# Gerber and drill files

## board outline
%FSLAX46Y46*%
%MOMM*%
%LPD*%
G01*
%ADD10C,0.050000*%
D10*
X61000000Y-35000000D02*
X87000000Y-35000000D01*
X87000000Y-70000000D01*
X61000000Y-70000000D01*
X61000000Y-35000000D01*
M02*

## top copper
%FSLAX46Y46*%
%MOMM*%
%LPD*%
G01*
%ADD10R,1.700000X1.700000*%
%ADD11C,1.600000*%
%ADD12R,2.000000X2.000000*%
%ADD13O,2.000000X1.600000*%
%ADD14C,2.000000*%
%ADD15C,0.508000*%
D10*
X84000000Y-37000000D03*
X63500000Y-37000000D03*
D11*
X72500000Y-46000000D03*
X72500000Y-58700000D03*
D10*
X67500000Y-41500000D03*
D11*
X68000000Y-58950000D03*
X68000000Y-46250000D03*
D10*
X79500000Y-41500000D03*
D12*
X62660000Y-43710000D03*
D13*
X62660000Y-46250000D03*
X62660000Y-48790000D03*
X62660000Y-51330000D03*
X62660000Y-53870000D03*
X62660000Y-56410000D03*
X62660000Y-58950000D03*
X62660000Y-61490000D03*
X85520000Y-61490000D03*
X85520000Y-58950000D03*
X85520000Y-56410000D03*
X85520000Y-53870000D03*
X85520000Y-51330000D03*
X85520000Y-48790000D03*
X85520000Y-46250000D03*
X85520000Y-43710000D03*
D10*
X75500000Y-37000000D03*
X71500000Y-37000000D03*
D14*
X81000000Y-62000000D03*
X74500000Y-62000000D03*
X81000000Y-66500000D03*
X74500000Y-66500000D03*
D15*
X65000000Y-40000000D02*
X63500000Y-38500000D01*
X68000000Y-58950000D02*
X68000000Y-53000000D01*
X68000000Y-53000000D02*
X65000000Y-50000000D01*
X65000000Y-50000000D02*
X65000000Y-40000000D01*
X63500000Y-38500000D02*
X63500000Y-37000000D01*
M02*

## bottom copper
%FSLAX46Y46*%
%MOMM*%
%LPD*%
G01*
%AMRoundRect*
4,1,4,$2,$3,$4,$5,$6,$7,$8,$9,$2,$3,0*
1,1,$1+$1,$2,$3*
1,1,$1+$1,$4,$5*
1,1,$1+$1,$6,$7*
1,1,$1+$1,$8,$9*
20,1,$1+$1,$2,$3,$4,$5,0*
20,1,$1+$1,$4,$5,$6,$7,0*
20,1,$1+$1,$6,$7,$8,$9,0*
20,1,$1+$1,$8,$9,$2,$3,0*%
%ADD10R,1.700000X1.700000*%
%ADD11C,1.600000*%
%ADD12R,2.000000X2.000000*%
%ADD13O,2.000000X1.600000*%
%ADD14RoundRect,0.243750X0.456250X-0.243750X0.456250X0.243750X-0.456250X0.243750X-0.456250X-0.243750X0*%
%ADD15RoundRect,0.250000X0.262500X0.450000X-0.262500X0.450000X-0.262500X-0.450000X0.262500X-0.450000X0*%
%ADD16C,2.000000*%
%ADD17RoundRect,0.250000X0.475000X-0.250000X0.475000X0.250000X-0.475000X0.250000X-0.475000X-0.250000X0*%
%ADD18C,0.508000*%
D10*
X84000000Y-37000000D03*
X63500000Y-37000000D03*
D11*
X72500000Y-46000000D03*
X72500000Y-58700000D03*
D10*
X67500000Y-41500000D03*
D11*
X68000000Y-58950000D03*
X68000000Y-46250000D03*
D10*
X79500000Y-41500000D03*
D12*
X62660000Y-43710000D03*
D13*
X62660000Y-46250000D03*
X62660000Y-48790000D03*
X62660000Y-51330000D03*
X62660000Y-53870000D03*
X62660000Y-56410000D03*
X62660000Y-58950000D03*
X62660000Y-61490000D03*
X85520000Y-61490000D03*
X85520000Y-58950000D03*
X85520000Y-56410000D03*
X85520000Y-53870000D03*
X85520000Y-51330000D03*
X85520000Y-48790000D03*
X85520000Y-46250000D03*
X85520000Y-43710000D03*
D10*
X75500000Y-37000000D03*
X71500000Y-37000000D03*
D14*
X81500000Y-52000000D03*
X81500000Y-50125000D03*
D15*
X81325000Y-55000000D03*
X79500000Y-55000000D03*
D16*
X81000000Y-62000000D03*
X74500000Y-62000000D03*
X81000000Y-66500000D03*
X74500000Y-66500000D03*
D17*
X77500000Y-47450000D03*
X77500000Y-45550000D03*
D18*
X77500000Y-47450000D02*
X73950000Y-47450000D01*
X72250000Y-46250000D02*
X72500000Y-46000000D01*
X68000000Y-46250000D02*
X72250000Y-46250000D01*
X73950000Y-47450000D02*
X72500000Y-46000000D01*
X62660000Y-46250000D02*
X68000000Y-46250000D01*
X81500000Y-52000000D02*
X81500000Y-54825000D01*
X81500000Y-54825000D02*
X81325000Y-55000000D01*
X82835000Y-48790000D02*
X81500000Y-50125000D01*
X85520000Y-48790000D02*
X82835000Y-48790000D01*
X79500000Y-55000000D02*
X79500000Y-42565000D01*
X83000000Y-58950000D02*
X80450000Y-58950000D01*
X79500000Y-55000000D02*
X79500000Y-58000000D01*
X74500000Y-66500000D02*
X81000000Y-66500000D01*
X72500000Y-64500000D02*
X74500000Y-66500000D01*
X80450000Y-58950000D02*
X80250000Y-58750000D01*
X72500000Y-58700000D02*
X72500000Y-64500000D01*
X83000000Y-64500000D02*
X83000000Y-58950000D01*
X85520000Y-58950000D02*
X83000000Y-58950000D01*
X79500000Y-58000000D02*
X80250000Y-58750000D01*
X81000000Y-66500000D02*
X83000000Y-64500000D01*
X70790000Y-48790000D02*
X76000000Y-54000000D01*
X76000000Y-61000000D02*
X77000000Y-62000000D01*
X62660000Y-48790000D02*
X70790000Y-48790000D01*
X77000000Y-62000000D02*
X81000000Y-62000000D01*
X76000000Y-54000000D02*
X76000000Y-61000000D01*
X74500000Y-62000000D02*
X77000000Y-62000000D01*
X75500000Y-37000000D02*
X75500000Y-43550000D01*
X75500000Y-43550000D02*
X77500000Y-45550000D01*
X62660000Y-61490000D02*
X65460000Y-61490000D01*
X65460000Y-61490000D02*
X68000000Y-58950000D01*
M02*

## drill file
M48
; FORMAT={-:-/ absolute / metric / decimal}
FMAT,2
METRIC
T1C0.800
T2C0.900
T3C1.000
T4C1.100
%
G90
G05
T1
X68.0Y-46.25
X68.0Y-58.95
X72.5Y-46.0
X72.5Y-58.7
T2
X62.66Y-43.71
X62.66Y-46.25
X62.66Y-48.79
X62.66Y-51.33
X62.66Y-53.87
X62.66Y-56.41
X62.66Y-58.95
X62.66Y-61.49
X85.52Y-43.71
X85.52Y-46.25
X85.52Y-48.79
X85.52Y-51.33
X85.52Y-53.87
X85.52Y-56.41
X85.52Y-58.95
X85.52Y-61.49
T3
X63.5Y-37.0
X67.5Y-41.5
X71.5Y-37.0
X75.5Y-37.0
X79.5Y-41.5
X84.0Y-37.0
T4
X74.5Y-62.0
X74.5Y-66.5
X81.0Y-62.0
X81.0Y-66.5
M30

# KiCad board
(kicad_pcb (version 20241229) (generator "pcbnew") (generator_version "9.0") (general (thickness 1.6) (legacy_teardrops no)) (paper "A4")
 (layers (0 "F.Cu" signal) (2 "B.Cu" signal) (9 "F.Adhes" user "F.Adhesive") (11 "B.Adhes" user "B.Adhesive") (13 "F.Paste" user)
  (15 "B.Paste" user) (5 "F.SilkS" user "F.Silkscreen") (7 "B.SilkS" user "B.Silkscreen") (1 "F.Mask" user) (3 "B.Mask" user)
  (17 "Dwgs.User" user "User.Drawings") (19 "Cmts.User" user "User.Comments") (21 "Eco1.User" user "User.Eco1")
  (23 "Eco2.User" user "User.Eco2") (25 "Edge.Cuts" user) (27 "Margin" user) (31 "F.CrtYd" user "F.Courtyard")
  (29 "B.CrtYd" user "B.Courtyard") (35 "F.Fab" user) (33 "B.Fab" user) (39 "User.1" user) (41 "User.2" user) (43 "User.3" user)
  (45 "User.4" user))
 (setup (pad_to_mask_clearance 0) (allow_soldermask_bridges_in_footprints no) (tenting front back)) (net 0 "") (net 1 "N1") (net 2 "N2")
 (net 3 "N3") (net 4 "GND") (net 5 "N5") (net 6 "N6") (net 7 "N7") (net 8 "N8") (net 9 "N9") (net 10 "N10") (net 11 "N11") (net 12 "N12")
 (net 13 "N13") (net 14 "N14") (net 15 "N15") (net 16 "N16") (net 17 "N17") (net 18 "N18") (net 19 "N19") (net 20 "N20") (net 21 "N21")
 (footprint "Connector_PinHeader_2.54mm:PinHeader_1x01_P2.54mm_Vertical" (layer "F.Cu") (at 84 37)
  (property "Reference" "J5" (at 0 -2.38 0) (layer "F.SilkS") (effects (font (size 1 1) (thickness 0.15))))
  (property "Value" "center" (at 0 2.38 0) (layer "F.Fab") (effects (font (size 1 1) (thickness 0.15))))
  (pad "1" thru_hole rect (at 0 0) (size 1.7 1.7) (drill 1) (layers "*.Cu" "*.Mask") (remove_unused_layers no) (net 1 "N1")))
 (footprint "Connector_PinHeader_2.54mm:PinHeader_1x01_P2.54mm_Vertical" (layer "F.Cu") (at 63.5 37)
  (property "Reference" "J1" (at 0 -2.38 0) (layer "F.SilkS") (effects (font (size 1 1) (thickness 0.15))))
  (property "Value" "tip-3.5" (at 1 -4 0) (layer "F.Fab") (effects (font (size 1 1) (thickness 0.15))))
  (pad "1" thru_hole rect (at 0 0) (size 1.7 1.7) (drill 1) (layers "*.Cu" "*.Mask") (remove_unused_layers no) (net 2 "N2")))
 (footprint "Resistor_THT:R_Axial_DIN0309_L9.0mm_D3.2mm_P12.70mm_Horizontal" (layer "F.Cu") (at 72.5 46 -90)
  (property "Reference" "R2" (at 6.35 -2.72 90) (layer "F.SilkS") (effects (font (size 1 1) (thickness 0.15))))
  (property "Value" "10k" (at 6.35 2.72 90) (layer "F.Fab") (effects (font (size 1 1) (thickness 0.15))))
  (pad "1" thru_hole circle (at 0 0 270) (size 1.6 1.6) (drill 0.8) (layers "*.Cu" "*.Mask") (remove_unused_layers no) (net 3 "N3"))
  (pad "2" thru_hole circle (at 12.7 0 270) (size 1.6 1.6) (drill 0.8) (layers "*.Cu" "*.Mask") (remove_unused_layers no) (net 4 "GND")))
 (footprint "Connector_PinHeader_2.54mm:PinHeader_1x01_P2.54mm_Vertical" (layer "F.Cu") (at 67.5 41.5)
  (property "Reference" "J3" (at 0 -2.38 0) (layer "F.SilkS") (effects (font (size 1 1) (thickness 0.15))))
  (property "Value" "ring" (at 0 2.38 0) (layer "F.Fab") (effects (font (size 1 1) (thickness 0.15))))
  (pad "1" thru_hole rect (at 0 0) (size 1.7 1.7) (drill 1) (layers "*.Cu" "*.Mask") (remove_unused_layers no) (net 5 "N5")))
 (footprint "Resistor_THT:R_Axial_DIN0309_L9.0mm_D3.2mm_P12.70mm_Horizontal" (layer "F.Cu") (at 68 58.95 90)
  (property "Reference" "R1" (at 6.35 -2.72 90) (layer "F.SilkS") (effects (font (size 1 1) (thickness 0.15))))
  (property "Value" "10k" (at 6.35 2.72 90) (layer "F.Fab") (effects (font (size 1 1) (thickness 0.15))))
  (pad "1" thru_hole circle (at 0 0 90) (size 1.6 1.6) (drill 0.8) (layers "*.Cu" "*.Mask") (remove_unused_layers no) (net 2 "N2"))
  (pad "2" thru_hole circle (at 12.7 0 90) (size 1.6 1.6) (drill 0.8) (layers "*.Cu" "*.Mask") (remove_unused_layers no) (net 3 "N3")))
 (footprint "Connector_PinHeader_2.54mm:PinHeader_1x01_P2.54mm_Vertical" (layer "F.Cu") (at 79.5 41.5)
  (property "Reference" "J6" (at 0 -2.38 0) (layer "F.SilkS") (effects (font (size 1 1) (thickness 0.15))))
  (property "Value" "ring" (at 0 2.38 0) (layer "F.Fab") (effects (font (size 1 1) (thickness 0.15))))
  (pad "1" thru_hole rect (at 0 0) (size 1.7 1.7) (drill 1) (layers "*.Cu" "*.Mask") (remove_unused_layers no) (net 4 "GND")))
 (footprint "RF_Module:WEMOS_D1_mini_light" (layer "F.Cu") (at 62.66 43.71)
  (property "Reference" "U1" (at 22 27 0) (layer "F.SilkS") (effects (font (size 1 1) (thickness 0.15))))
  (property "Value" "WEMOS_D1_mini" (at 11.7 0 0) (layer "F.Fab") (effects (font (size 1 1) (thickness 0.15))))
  (pad "1" thru_hole rect (at 0 0) (size 2 2) (drill 0.9) (layers "*.Cu" "*.Mask") (remove_unused_layers no) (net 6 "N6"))
  (pad "2" thru_hole oval (at 0 2.54) (size 2 1.6) (drill 0.9) (layers "*.Cu" "*.Mask") (remove_unused_layers no) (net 3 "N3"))
  (pad "3" thru_hole oval (at 0 5.08) (size 2 1.6) (drill 0.9) (layers "*.Cu" "*.Mask") (remove_unused_layers no) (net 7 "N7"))
  (pad "4" thru_hole oval (at 0 7.62) (size 2 1.6) (drill 0.9) (layers "*.Cu" "*.Mask") (remove_unused_layers no) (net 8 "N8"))
  (pad "5" thru_hole oval (at 0 10.16) (size 2 1.6) (drill 0.9) (layers "*.Cu" "*.Mask") (remove_unused_layers no) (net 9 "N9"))
  (pad "6" thru_hole oval (at 0 12.7) (size 2 1.6) (drill 0.9) (layers "*.Cu" "*.Mask") (remove_unused_layers no) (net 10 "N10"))
  (pad "7" thru_hole oval (at 0 15.24) (size 2 1.6) (drill 0.9) (layers "*.Cu" "*.Mask") (remove_unused_layers no) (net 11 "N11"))
  (pad "8" thru_hole oval (at 0 17.78) (size 2 1.6) (drill 0.9) (layers "*.Cu" "*.Mask") (remove_unused_layers no) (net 2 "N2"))
  (pad "9" thru_hole oval (at 22.86 17.78) (size 2 1.6) (drill 0.9) (layers "*.Cu" "*.Mask") (remove_unused_layers no) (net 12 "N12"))
  (pad "10" thru_hole oval (at 22.86 15.24) (size 2 1.6) (drill 0.9) (layers "*.Cu" "*.Mask") (remove_unused_layers no) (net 4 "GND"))
  (pad "11" thru_hole oval (at 22.86 12.7) (size 2 1.6) (drill 0.9) (layers "*.Cu" "*.Mask") (remove_unused_layers no) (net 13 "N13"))
  (pad "12" thru_hole oval (at 22.86 10.16) (size 2 1.6) (drill 0.9) (layers "*.Cu" "*.Mask") (remove_unused_layers no) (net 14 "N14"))
  (pad "13" thru_hole oval (at 22.86 7.62) (size 2 1.6) (drill 0.9) (layers "*.Cu" "*.Mask") (remove_unused_layers no) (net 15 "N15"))
  (pad "14" thru_hole oval (at 22.86 5.08) (size 2 1.6) (drill 0.9) (layers "*.Cu" "*.Mask") (remove_unused_layers no) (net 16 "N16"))
  (pad "15" thru_hole oval (at 22.86 2.54) (size 2 1.6) (drill 0.9) (layers "*.Cu" "*.Mask") (remove_unused_layers no) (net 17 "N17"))
  (pad "16" thru_hole oval (at 22.86 0) (size 2 1.6) (drill 0.9) (layers "*.Cu" "*.Mask") (remove_unused_layers no) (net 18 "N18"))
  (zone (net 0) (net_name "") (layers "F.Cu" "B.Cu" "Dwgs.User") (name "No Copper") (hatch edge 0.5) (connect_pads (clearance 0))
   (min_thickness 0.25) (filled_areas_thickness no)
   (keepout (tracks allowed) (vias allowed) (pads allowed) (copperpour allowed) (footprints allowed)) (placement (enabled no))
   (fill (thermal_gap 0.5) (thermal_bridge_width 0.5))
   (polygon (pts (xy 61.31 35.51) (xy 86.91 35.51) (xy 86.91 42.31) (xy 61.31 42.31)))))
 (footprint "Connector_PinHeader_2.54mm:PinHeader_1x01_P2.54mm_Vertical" (layer "F.Cu") (at 75.5 37)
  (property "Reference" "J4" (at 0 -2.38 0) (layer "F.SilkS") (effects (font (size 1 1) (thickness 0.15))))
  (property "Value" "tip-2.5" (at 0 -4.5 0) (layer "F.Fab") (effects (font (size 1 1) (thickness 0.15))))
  (pad "1" thru_hole rect (at 0 0) (size 1.7 1.7) (drill 1) (layers "*.Cu" "*.Mask") (remove_unused_layers no) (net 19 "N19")))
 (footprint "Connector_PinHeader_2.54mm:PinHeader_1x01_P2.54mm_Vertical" (layer "F.Cu") (at 71.5 37)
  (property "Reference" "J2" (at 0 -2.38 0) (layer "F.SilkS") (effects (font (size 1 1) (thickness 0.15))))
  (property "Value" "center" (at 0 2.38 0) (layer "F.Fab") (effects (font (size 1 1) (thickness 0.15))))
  (pad "1" thru_hole rect (at 0 0) (size 1.7 1.7) (drill 1) (layers "*.Cu" "*.Mask") (remove_unused_layers no) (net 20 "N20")))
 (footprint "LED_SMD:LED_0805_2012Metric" (layer "B.Cu") (at 81.5 51.0625 90)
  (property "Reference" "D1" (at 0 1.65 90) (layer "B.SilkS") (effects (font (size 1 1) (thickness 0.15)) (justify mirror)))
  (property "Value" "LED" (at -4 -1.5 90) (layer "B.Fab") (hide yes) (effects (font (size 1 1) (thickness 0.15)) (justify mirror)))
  (pad "1" smd roundrect (at -0.9375 0 90) (size 0.975 1.4) (layers "B.Cu" "B.Mask" "B.Paste") (roundrect_rratio 0.25) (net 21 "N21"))
  (pad "2" smd roundrect (at 0.9375 0 90) (size 0.975 1.4) (layers "B.Cu" "B.Mask" "B.Paste") (roundrect_rratio 0.25) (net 16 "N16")))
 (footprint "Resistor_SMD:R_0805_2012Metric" (layer "B.Cu") (at 80.4125 55 180)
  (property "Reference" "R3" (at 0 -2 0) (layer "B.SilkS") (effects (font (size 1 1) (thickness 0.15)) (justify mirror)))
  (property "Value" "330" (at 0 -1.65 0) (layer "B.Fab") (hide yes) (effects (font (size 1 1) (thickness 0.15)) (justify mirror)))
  (pad "1" smd roundrect (at -0.9125 0 180) (size 1.025 1.4) (layers "B.Cu" "B.Mask" "B.Paste") (roundrect_rratio 0.243902) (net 21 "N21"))
  (pad "2" smd roundrect (at 0.9125 0 180) (size 1.025 1.4) (layers "B.Cu" "B.Mask" "B.Paste") (roundrect_rratio 0.243902) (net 4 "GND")))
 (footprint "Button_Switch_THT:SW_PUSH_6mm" (layer "B.Cu") (at 81 62 180)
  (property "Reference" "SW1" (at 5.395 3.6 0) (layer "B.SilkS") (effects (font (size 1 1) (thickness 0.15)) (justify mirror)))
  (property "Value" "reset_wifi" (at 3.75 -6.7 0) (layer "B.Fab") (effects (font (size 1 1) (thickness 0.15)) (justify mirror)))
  (pad "1" thru_hole circle (at 0 0 90) (size 2 2) (drill 1.1) (layers "*.Cu" "*.Mask") (remove_unused_layers no) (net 7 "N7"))
  (pad "1" thru_hole circle (at 6.5 0 90) (size 2 2) (drill 1.1) (layers "*.Cu" "*.Mask") (remove_unused_layers no) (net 7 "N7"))
  (pad "2" thru_hole circle (at 0 -4.5 90) (size 2 2) (drill 1.1) (layers "*.Cu" "*.Mask") (remove_unused_layers no) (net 4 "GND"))
  (pad "2" thru_hole circle (at 6.5 -4.5 90) (size 2 2) (drill 1.1) (layers "*.Cu" "*.Mask") (remove_unused_layers no) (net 4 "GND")))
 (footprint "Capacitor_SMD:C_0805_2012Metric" (layer "B.Cu") (at 77.5 46.5 90)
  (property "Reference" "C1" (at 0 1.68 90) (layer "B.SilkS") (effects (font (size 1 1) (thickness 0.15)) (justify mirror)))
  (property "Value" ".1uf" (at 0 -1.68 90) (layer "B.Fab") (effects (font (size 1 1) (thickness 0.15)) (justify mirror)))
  (pad "1" smd roundrect (at -0.95 0 90) (size 1 1.45) (layers "B.Cu" "B.Mask" "B.Paste") (roundrect_rratio 0.25) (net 3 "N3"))
  (pad "2" smd roundrect (at 0.95 0 90) (size 1 1.45) (layers "B.Cu" "B.Mask" "B.Paste") (roundrect_rratio 0.25) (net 19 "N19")))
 (gr_rect (start 61 35) (end 87 70) (stroke (width 0.05) (type default)) (fill no) (layer "Edge.Cuts"))
 (segment (start 77.5 47.45) (end 73.95 47.45) (width 0.508) (layer "B.Cu") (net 3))
 (segment (start 72.25 46.25) (end 72.5 46) (width 0.508) (layer "B.Cu") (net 3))
 (segment (start 68 46.25) (end 72.25 46.25) (width 0.508) (layer "B.Cu") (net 3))
 (segment (start 73.95 47.45) (end 72.5 46) (width 0.508) (layer "B.Cu") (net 3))
 (segment (start 62.66 46.25) (end 68 46.25) (width 0.508) (layer "B.Cu") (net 3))
 (segment (start 81.5 52) (end 81.5 54.825) (width 0.508) (layer "B.Cu") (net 21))
 (segment (start 81.5 54.825) (end 81.325 55) (width 0.508) (layer "B.Cu") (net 21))
 (segment (start 82.835 48.79) (end 81.5 50.125) (width 0.508) (layer "B.Cu") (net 16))
 (segment (start 85.52 48.79) (end 82.835 48.79) (width 0.508) (layer "B.Cu") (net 16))
 (segment (start 79.5 55) (end 79.5 42.565) (width 0.508) (layer "B.Cu") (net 4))
 (segment (start 83 58.95) (end 80.45 58.95) (width 0.508) (layer "B.Cu") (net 4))
 (segment (start 79.5 55) (end 79.5 58) (width 0.508) (layer "B.Cu") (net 4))
 (segment (start 74.5 66.5) (end 81 66.5) (width 0.508) (layer "B.Cu") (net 4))
 (segment (start 72.5 64.5) (end 74.5 66.5) (width 0.508) (layer "B.Cu") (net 4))
 (segment (start 80.45 58.95) (end 80.25 58.75) (width 0.508) (layer "B.Cu") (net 4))
 (segment (start 72.5 58.7) (end 72.5 64.5) (width 0.508) (layer "B.Cu") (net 4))
 (segment (start 83 64.5) (end 83 58.95) (width 0.508) (layer "B.Cu") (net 4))
 (segment (start 85.52 58.95) (end 83 58.95) (width 0.508) (layer "B.Cu") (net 4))
 (segment (start 79.5 58) (end 80.25 58.75) (width 0.508) (layer "B.Cu") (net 4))
 (segment (start 81 66.5) (end 83 64.5) (width 0.508) (layer "B.Cu") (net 4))
 (segment (start 70.79 48.79) (end 76 54) (width 0.508) (layer "B.Cu") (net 7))
 (segment (start 76 61) (end 77 62) (width 0.508) (layer "B.Cu") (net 7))
 (segment (start 62.66 48.79) (end 70.79 48.79) (width 0.508) (layer "B.Cu") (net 7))
 (segment (start 77 62) (end 81 62) (width 0.508) (layer "B.Cu") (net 7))
 (segment (start 76 54) (end 76 61) (width 0.508) (layer "B.Cu") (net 7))
 (segment (start 74.5 62) (end 77 62) (width 0.508) (layer "B.Cu") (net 7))
 (segment (start 75.5 37) (end 75.5 43.55) (width 0.508) (layer "B.Cu") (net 19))
 (segment (start 75.5 43.55) (end 77.5 45.55) (width 0.508) (layer "B.Cu") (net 19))
 (segment (start 65 40) (end 63.5 38.5) (width 0.508) (layer "F.Cu") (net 2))
 (segment (start 68 58.95) (end 68 53) (width 0.508) (layer "F.Cu") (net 2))
 (segment (start 68 53) (end 65 50) (width 0.508) (layer "F.Cu") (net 2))
 (segment (start 65 50) (end 65 40) (width 0.508) (layer "F.Cu") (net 2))
 (segment (start 63.5 38.5) (end 63.5 37) (width 0.508) (layer "F.Cu") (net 2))
 (segment (start 62.66 61.49) (end 65.46 61.49) (width 0.508) (layer "B.Cu") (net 2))
 (segment (start 65.46 61.49) (end 68 58.95) (width 0.508) (layer "B.Cu") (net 2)))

